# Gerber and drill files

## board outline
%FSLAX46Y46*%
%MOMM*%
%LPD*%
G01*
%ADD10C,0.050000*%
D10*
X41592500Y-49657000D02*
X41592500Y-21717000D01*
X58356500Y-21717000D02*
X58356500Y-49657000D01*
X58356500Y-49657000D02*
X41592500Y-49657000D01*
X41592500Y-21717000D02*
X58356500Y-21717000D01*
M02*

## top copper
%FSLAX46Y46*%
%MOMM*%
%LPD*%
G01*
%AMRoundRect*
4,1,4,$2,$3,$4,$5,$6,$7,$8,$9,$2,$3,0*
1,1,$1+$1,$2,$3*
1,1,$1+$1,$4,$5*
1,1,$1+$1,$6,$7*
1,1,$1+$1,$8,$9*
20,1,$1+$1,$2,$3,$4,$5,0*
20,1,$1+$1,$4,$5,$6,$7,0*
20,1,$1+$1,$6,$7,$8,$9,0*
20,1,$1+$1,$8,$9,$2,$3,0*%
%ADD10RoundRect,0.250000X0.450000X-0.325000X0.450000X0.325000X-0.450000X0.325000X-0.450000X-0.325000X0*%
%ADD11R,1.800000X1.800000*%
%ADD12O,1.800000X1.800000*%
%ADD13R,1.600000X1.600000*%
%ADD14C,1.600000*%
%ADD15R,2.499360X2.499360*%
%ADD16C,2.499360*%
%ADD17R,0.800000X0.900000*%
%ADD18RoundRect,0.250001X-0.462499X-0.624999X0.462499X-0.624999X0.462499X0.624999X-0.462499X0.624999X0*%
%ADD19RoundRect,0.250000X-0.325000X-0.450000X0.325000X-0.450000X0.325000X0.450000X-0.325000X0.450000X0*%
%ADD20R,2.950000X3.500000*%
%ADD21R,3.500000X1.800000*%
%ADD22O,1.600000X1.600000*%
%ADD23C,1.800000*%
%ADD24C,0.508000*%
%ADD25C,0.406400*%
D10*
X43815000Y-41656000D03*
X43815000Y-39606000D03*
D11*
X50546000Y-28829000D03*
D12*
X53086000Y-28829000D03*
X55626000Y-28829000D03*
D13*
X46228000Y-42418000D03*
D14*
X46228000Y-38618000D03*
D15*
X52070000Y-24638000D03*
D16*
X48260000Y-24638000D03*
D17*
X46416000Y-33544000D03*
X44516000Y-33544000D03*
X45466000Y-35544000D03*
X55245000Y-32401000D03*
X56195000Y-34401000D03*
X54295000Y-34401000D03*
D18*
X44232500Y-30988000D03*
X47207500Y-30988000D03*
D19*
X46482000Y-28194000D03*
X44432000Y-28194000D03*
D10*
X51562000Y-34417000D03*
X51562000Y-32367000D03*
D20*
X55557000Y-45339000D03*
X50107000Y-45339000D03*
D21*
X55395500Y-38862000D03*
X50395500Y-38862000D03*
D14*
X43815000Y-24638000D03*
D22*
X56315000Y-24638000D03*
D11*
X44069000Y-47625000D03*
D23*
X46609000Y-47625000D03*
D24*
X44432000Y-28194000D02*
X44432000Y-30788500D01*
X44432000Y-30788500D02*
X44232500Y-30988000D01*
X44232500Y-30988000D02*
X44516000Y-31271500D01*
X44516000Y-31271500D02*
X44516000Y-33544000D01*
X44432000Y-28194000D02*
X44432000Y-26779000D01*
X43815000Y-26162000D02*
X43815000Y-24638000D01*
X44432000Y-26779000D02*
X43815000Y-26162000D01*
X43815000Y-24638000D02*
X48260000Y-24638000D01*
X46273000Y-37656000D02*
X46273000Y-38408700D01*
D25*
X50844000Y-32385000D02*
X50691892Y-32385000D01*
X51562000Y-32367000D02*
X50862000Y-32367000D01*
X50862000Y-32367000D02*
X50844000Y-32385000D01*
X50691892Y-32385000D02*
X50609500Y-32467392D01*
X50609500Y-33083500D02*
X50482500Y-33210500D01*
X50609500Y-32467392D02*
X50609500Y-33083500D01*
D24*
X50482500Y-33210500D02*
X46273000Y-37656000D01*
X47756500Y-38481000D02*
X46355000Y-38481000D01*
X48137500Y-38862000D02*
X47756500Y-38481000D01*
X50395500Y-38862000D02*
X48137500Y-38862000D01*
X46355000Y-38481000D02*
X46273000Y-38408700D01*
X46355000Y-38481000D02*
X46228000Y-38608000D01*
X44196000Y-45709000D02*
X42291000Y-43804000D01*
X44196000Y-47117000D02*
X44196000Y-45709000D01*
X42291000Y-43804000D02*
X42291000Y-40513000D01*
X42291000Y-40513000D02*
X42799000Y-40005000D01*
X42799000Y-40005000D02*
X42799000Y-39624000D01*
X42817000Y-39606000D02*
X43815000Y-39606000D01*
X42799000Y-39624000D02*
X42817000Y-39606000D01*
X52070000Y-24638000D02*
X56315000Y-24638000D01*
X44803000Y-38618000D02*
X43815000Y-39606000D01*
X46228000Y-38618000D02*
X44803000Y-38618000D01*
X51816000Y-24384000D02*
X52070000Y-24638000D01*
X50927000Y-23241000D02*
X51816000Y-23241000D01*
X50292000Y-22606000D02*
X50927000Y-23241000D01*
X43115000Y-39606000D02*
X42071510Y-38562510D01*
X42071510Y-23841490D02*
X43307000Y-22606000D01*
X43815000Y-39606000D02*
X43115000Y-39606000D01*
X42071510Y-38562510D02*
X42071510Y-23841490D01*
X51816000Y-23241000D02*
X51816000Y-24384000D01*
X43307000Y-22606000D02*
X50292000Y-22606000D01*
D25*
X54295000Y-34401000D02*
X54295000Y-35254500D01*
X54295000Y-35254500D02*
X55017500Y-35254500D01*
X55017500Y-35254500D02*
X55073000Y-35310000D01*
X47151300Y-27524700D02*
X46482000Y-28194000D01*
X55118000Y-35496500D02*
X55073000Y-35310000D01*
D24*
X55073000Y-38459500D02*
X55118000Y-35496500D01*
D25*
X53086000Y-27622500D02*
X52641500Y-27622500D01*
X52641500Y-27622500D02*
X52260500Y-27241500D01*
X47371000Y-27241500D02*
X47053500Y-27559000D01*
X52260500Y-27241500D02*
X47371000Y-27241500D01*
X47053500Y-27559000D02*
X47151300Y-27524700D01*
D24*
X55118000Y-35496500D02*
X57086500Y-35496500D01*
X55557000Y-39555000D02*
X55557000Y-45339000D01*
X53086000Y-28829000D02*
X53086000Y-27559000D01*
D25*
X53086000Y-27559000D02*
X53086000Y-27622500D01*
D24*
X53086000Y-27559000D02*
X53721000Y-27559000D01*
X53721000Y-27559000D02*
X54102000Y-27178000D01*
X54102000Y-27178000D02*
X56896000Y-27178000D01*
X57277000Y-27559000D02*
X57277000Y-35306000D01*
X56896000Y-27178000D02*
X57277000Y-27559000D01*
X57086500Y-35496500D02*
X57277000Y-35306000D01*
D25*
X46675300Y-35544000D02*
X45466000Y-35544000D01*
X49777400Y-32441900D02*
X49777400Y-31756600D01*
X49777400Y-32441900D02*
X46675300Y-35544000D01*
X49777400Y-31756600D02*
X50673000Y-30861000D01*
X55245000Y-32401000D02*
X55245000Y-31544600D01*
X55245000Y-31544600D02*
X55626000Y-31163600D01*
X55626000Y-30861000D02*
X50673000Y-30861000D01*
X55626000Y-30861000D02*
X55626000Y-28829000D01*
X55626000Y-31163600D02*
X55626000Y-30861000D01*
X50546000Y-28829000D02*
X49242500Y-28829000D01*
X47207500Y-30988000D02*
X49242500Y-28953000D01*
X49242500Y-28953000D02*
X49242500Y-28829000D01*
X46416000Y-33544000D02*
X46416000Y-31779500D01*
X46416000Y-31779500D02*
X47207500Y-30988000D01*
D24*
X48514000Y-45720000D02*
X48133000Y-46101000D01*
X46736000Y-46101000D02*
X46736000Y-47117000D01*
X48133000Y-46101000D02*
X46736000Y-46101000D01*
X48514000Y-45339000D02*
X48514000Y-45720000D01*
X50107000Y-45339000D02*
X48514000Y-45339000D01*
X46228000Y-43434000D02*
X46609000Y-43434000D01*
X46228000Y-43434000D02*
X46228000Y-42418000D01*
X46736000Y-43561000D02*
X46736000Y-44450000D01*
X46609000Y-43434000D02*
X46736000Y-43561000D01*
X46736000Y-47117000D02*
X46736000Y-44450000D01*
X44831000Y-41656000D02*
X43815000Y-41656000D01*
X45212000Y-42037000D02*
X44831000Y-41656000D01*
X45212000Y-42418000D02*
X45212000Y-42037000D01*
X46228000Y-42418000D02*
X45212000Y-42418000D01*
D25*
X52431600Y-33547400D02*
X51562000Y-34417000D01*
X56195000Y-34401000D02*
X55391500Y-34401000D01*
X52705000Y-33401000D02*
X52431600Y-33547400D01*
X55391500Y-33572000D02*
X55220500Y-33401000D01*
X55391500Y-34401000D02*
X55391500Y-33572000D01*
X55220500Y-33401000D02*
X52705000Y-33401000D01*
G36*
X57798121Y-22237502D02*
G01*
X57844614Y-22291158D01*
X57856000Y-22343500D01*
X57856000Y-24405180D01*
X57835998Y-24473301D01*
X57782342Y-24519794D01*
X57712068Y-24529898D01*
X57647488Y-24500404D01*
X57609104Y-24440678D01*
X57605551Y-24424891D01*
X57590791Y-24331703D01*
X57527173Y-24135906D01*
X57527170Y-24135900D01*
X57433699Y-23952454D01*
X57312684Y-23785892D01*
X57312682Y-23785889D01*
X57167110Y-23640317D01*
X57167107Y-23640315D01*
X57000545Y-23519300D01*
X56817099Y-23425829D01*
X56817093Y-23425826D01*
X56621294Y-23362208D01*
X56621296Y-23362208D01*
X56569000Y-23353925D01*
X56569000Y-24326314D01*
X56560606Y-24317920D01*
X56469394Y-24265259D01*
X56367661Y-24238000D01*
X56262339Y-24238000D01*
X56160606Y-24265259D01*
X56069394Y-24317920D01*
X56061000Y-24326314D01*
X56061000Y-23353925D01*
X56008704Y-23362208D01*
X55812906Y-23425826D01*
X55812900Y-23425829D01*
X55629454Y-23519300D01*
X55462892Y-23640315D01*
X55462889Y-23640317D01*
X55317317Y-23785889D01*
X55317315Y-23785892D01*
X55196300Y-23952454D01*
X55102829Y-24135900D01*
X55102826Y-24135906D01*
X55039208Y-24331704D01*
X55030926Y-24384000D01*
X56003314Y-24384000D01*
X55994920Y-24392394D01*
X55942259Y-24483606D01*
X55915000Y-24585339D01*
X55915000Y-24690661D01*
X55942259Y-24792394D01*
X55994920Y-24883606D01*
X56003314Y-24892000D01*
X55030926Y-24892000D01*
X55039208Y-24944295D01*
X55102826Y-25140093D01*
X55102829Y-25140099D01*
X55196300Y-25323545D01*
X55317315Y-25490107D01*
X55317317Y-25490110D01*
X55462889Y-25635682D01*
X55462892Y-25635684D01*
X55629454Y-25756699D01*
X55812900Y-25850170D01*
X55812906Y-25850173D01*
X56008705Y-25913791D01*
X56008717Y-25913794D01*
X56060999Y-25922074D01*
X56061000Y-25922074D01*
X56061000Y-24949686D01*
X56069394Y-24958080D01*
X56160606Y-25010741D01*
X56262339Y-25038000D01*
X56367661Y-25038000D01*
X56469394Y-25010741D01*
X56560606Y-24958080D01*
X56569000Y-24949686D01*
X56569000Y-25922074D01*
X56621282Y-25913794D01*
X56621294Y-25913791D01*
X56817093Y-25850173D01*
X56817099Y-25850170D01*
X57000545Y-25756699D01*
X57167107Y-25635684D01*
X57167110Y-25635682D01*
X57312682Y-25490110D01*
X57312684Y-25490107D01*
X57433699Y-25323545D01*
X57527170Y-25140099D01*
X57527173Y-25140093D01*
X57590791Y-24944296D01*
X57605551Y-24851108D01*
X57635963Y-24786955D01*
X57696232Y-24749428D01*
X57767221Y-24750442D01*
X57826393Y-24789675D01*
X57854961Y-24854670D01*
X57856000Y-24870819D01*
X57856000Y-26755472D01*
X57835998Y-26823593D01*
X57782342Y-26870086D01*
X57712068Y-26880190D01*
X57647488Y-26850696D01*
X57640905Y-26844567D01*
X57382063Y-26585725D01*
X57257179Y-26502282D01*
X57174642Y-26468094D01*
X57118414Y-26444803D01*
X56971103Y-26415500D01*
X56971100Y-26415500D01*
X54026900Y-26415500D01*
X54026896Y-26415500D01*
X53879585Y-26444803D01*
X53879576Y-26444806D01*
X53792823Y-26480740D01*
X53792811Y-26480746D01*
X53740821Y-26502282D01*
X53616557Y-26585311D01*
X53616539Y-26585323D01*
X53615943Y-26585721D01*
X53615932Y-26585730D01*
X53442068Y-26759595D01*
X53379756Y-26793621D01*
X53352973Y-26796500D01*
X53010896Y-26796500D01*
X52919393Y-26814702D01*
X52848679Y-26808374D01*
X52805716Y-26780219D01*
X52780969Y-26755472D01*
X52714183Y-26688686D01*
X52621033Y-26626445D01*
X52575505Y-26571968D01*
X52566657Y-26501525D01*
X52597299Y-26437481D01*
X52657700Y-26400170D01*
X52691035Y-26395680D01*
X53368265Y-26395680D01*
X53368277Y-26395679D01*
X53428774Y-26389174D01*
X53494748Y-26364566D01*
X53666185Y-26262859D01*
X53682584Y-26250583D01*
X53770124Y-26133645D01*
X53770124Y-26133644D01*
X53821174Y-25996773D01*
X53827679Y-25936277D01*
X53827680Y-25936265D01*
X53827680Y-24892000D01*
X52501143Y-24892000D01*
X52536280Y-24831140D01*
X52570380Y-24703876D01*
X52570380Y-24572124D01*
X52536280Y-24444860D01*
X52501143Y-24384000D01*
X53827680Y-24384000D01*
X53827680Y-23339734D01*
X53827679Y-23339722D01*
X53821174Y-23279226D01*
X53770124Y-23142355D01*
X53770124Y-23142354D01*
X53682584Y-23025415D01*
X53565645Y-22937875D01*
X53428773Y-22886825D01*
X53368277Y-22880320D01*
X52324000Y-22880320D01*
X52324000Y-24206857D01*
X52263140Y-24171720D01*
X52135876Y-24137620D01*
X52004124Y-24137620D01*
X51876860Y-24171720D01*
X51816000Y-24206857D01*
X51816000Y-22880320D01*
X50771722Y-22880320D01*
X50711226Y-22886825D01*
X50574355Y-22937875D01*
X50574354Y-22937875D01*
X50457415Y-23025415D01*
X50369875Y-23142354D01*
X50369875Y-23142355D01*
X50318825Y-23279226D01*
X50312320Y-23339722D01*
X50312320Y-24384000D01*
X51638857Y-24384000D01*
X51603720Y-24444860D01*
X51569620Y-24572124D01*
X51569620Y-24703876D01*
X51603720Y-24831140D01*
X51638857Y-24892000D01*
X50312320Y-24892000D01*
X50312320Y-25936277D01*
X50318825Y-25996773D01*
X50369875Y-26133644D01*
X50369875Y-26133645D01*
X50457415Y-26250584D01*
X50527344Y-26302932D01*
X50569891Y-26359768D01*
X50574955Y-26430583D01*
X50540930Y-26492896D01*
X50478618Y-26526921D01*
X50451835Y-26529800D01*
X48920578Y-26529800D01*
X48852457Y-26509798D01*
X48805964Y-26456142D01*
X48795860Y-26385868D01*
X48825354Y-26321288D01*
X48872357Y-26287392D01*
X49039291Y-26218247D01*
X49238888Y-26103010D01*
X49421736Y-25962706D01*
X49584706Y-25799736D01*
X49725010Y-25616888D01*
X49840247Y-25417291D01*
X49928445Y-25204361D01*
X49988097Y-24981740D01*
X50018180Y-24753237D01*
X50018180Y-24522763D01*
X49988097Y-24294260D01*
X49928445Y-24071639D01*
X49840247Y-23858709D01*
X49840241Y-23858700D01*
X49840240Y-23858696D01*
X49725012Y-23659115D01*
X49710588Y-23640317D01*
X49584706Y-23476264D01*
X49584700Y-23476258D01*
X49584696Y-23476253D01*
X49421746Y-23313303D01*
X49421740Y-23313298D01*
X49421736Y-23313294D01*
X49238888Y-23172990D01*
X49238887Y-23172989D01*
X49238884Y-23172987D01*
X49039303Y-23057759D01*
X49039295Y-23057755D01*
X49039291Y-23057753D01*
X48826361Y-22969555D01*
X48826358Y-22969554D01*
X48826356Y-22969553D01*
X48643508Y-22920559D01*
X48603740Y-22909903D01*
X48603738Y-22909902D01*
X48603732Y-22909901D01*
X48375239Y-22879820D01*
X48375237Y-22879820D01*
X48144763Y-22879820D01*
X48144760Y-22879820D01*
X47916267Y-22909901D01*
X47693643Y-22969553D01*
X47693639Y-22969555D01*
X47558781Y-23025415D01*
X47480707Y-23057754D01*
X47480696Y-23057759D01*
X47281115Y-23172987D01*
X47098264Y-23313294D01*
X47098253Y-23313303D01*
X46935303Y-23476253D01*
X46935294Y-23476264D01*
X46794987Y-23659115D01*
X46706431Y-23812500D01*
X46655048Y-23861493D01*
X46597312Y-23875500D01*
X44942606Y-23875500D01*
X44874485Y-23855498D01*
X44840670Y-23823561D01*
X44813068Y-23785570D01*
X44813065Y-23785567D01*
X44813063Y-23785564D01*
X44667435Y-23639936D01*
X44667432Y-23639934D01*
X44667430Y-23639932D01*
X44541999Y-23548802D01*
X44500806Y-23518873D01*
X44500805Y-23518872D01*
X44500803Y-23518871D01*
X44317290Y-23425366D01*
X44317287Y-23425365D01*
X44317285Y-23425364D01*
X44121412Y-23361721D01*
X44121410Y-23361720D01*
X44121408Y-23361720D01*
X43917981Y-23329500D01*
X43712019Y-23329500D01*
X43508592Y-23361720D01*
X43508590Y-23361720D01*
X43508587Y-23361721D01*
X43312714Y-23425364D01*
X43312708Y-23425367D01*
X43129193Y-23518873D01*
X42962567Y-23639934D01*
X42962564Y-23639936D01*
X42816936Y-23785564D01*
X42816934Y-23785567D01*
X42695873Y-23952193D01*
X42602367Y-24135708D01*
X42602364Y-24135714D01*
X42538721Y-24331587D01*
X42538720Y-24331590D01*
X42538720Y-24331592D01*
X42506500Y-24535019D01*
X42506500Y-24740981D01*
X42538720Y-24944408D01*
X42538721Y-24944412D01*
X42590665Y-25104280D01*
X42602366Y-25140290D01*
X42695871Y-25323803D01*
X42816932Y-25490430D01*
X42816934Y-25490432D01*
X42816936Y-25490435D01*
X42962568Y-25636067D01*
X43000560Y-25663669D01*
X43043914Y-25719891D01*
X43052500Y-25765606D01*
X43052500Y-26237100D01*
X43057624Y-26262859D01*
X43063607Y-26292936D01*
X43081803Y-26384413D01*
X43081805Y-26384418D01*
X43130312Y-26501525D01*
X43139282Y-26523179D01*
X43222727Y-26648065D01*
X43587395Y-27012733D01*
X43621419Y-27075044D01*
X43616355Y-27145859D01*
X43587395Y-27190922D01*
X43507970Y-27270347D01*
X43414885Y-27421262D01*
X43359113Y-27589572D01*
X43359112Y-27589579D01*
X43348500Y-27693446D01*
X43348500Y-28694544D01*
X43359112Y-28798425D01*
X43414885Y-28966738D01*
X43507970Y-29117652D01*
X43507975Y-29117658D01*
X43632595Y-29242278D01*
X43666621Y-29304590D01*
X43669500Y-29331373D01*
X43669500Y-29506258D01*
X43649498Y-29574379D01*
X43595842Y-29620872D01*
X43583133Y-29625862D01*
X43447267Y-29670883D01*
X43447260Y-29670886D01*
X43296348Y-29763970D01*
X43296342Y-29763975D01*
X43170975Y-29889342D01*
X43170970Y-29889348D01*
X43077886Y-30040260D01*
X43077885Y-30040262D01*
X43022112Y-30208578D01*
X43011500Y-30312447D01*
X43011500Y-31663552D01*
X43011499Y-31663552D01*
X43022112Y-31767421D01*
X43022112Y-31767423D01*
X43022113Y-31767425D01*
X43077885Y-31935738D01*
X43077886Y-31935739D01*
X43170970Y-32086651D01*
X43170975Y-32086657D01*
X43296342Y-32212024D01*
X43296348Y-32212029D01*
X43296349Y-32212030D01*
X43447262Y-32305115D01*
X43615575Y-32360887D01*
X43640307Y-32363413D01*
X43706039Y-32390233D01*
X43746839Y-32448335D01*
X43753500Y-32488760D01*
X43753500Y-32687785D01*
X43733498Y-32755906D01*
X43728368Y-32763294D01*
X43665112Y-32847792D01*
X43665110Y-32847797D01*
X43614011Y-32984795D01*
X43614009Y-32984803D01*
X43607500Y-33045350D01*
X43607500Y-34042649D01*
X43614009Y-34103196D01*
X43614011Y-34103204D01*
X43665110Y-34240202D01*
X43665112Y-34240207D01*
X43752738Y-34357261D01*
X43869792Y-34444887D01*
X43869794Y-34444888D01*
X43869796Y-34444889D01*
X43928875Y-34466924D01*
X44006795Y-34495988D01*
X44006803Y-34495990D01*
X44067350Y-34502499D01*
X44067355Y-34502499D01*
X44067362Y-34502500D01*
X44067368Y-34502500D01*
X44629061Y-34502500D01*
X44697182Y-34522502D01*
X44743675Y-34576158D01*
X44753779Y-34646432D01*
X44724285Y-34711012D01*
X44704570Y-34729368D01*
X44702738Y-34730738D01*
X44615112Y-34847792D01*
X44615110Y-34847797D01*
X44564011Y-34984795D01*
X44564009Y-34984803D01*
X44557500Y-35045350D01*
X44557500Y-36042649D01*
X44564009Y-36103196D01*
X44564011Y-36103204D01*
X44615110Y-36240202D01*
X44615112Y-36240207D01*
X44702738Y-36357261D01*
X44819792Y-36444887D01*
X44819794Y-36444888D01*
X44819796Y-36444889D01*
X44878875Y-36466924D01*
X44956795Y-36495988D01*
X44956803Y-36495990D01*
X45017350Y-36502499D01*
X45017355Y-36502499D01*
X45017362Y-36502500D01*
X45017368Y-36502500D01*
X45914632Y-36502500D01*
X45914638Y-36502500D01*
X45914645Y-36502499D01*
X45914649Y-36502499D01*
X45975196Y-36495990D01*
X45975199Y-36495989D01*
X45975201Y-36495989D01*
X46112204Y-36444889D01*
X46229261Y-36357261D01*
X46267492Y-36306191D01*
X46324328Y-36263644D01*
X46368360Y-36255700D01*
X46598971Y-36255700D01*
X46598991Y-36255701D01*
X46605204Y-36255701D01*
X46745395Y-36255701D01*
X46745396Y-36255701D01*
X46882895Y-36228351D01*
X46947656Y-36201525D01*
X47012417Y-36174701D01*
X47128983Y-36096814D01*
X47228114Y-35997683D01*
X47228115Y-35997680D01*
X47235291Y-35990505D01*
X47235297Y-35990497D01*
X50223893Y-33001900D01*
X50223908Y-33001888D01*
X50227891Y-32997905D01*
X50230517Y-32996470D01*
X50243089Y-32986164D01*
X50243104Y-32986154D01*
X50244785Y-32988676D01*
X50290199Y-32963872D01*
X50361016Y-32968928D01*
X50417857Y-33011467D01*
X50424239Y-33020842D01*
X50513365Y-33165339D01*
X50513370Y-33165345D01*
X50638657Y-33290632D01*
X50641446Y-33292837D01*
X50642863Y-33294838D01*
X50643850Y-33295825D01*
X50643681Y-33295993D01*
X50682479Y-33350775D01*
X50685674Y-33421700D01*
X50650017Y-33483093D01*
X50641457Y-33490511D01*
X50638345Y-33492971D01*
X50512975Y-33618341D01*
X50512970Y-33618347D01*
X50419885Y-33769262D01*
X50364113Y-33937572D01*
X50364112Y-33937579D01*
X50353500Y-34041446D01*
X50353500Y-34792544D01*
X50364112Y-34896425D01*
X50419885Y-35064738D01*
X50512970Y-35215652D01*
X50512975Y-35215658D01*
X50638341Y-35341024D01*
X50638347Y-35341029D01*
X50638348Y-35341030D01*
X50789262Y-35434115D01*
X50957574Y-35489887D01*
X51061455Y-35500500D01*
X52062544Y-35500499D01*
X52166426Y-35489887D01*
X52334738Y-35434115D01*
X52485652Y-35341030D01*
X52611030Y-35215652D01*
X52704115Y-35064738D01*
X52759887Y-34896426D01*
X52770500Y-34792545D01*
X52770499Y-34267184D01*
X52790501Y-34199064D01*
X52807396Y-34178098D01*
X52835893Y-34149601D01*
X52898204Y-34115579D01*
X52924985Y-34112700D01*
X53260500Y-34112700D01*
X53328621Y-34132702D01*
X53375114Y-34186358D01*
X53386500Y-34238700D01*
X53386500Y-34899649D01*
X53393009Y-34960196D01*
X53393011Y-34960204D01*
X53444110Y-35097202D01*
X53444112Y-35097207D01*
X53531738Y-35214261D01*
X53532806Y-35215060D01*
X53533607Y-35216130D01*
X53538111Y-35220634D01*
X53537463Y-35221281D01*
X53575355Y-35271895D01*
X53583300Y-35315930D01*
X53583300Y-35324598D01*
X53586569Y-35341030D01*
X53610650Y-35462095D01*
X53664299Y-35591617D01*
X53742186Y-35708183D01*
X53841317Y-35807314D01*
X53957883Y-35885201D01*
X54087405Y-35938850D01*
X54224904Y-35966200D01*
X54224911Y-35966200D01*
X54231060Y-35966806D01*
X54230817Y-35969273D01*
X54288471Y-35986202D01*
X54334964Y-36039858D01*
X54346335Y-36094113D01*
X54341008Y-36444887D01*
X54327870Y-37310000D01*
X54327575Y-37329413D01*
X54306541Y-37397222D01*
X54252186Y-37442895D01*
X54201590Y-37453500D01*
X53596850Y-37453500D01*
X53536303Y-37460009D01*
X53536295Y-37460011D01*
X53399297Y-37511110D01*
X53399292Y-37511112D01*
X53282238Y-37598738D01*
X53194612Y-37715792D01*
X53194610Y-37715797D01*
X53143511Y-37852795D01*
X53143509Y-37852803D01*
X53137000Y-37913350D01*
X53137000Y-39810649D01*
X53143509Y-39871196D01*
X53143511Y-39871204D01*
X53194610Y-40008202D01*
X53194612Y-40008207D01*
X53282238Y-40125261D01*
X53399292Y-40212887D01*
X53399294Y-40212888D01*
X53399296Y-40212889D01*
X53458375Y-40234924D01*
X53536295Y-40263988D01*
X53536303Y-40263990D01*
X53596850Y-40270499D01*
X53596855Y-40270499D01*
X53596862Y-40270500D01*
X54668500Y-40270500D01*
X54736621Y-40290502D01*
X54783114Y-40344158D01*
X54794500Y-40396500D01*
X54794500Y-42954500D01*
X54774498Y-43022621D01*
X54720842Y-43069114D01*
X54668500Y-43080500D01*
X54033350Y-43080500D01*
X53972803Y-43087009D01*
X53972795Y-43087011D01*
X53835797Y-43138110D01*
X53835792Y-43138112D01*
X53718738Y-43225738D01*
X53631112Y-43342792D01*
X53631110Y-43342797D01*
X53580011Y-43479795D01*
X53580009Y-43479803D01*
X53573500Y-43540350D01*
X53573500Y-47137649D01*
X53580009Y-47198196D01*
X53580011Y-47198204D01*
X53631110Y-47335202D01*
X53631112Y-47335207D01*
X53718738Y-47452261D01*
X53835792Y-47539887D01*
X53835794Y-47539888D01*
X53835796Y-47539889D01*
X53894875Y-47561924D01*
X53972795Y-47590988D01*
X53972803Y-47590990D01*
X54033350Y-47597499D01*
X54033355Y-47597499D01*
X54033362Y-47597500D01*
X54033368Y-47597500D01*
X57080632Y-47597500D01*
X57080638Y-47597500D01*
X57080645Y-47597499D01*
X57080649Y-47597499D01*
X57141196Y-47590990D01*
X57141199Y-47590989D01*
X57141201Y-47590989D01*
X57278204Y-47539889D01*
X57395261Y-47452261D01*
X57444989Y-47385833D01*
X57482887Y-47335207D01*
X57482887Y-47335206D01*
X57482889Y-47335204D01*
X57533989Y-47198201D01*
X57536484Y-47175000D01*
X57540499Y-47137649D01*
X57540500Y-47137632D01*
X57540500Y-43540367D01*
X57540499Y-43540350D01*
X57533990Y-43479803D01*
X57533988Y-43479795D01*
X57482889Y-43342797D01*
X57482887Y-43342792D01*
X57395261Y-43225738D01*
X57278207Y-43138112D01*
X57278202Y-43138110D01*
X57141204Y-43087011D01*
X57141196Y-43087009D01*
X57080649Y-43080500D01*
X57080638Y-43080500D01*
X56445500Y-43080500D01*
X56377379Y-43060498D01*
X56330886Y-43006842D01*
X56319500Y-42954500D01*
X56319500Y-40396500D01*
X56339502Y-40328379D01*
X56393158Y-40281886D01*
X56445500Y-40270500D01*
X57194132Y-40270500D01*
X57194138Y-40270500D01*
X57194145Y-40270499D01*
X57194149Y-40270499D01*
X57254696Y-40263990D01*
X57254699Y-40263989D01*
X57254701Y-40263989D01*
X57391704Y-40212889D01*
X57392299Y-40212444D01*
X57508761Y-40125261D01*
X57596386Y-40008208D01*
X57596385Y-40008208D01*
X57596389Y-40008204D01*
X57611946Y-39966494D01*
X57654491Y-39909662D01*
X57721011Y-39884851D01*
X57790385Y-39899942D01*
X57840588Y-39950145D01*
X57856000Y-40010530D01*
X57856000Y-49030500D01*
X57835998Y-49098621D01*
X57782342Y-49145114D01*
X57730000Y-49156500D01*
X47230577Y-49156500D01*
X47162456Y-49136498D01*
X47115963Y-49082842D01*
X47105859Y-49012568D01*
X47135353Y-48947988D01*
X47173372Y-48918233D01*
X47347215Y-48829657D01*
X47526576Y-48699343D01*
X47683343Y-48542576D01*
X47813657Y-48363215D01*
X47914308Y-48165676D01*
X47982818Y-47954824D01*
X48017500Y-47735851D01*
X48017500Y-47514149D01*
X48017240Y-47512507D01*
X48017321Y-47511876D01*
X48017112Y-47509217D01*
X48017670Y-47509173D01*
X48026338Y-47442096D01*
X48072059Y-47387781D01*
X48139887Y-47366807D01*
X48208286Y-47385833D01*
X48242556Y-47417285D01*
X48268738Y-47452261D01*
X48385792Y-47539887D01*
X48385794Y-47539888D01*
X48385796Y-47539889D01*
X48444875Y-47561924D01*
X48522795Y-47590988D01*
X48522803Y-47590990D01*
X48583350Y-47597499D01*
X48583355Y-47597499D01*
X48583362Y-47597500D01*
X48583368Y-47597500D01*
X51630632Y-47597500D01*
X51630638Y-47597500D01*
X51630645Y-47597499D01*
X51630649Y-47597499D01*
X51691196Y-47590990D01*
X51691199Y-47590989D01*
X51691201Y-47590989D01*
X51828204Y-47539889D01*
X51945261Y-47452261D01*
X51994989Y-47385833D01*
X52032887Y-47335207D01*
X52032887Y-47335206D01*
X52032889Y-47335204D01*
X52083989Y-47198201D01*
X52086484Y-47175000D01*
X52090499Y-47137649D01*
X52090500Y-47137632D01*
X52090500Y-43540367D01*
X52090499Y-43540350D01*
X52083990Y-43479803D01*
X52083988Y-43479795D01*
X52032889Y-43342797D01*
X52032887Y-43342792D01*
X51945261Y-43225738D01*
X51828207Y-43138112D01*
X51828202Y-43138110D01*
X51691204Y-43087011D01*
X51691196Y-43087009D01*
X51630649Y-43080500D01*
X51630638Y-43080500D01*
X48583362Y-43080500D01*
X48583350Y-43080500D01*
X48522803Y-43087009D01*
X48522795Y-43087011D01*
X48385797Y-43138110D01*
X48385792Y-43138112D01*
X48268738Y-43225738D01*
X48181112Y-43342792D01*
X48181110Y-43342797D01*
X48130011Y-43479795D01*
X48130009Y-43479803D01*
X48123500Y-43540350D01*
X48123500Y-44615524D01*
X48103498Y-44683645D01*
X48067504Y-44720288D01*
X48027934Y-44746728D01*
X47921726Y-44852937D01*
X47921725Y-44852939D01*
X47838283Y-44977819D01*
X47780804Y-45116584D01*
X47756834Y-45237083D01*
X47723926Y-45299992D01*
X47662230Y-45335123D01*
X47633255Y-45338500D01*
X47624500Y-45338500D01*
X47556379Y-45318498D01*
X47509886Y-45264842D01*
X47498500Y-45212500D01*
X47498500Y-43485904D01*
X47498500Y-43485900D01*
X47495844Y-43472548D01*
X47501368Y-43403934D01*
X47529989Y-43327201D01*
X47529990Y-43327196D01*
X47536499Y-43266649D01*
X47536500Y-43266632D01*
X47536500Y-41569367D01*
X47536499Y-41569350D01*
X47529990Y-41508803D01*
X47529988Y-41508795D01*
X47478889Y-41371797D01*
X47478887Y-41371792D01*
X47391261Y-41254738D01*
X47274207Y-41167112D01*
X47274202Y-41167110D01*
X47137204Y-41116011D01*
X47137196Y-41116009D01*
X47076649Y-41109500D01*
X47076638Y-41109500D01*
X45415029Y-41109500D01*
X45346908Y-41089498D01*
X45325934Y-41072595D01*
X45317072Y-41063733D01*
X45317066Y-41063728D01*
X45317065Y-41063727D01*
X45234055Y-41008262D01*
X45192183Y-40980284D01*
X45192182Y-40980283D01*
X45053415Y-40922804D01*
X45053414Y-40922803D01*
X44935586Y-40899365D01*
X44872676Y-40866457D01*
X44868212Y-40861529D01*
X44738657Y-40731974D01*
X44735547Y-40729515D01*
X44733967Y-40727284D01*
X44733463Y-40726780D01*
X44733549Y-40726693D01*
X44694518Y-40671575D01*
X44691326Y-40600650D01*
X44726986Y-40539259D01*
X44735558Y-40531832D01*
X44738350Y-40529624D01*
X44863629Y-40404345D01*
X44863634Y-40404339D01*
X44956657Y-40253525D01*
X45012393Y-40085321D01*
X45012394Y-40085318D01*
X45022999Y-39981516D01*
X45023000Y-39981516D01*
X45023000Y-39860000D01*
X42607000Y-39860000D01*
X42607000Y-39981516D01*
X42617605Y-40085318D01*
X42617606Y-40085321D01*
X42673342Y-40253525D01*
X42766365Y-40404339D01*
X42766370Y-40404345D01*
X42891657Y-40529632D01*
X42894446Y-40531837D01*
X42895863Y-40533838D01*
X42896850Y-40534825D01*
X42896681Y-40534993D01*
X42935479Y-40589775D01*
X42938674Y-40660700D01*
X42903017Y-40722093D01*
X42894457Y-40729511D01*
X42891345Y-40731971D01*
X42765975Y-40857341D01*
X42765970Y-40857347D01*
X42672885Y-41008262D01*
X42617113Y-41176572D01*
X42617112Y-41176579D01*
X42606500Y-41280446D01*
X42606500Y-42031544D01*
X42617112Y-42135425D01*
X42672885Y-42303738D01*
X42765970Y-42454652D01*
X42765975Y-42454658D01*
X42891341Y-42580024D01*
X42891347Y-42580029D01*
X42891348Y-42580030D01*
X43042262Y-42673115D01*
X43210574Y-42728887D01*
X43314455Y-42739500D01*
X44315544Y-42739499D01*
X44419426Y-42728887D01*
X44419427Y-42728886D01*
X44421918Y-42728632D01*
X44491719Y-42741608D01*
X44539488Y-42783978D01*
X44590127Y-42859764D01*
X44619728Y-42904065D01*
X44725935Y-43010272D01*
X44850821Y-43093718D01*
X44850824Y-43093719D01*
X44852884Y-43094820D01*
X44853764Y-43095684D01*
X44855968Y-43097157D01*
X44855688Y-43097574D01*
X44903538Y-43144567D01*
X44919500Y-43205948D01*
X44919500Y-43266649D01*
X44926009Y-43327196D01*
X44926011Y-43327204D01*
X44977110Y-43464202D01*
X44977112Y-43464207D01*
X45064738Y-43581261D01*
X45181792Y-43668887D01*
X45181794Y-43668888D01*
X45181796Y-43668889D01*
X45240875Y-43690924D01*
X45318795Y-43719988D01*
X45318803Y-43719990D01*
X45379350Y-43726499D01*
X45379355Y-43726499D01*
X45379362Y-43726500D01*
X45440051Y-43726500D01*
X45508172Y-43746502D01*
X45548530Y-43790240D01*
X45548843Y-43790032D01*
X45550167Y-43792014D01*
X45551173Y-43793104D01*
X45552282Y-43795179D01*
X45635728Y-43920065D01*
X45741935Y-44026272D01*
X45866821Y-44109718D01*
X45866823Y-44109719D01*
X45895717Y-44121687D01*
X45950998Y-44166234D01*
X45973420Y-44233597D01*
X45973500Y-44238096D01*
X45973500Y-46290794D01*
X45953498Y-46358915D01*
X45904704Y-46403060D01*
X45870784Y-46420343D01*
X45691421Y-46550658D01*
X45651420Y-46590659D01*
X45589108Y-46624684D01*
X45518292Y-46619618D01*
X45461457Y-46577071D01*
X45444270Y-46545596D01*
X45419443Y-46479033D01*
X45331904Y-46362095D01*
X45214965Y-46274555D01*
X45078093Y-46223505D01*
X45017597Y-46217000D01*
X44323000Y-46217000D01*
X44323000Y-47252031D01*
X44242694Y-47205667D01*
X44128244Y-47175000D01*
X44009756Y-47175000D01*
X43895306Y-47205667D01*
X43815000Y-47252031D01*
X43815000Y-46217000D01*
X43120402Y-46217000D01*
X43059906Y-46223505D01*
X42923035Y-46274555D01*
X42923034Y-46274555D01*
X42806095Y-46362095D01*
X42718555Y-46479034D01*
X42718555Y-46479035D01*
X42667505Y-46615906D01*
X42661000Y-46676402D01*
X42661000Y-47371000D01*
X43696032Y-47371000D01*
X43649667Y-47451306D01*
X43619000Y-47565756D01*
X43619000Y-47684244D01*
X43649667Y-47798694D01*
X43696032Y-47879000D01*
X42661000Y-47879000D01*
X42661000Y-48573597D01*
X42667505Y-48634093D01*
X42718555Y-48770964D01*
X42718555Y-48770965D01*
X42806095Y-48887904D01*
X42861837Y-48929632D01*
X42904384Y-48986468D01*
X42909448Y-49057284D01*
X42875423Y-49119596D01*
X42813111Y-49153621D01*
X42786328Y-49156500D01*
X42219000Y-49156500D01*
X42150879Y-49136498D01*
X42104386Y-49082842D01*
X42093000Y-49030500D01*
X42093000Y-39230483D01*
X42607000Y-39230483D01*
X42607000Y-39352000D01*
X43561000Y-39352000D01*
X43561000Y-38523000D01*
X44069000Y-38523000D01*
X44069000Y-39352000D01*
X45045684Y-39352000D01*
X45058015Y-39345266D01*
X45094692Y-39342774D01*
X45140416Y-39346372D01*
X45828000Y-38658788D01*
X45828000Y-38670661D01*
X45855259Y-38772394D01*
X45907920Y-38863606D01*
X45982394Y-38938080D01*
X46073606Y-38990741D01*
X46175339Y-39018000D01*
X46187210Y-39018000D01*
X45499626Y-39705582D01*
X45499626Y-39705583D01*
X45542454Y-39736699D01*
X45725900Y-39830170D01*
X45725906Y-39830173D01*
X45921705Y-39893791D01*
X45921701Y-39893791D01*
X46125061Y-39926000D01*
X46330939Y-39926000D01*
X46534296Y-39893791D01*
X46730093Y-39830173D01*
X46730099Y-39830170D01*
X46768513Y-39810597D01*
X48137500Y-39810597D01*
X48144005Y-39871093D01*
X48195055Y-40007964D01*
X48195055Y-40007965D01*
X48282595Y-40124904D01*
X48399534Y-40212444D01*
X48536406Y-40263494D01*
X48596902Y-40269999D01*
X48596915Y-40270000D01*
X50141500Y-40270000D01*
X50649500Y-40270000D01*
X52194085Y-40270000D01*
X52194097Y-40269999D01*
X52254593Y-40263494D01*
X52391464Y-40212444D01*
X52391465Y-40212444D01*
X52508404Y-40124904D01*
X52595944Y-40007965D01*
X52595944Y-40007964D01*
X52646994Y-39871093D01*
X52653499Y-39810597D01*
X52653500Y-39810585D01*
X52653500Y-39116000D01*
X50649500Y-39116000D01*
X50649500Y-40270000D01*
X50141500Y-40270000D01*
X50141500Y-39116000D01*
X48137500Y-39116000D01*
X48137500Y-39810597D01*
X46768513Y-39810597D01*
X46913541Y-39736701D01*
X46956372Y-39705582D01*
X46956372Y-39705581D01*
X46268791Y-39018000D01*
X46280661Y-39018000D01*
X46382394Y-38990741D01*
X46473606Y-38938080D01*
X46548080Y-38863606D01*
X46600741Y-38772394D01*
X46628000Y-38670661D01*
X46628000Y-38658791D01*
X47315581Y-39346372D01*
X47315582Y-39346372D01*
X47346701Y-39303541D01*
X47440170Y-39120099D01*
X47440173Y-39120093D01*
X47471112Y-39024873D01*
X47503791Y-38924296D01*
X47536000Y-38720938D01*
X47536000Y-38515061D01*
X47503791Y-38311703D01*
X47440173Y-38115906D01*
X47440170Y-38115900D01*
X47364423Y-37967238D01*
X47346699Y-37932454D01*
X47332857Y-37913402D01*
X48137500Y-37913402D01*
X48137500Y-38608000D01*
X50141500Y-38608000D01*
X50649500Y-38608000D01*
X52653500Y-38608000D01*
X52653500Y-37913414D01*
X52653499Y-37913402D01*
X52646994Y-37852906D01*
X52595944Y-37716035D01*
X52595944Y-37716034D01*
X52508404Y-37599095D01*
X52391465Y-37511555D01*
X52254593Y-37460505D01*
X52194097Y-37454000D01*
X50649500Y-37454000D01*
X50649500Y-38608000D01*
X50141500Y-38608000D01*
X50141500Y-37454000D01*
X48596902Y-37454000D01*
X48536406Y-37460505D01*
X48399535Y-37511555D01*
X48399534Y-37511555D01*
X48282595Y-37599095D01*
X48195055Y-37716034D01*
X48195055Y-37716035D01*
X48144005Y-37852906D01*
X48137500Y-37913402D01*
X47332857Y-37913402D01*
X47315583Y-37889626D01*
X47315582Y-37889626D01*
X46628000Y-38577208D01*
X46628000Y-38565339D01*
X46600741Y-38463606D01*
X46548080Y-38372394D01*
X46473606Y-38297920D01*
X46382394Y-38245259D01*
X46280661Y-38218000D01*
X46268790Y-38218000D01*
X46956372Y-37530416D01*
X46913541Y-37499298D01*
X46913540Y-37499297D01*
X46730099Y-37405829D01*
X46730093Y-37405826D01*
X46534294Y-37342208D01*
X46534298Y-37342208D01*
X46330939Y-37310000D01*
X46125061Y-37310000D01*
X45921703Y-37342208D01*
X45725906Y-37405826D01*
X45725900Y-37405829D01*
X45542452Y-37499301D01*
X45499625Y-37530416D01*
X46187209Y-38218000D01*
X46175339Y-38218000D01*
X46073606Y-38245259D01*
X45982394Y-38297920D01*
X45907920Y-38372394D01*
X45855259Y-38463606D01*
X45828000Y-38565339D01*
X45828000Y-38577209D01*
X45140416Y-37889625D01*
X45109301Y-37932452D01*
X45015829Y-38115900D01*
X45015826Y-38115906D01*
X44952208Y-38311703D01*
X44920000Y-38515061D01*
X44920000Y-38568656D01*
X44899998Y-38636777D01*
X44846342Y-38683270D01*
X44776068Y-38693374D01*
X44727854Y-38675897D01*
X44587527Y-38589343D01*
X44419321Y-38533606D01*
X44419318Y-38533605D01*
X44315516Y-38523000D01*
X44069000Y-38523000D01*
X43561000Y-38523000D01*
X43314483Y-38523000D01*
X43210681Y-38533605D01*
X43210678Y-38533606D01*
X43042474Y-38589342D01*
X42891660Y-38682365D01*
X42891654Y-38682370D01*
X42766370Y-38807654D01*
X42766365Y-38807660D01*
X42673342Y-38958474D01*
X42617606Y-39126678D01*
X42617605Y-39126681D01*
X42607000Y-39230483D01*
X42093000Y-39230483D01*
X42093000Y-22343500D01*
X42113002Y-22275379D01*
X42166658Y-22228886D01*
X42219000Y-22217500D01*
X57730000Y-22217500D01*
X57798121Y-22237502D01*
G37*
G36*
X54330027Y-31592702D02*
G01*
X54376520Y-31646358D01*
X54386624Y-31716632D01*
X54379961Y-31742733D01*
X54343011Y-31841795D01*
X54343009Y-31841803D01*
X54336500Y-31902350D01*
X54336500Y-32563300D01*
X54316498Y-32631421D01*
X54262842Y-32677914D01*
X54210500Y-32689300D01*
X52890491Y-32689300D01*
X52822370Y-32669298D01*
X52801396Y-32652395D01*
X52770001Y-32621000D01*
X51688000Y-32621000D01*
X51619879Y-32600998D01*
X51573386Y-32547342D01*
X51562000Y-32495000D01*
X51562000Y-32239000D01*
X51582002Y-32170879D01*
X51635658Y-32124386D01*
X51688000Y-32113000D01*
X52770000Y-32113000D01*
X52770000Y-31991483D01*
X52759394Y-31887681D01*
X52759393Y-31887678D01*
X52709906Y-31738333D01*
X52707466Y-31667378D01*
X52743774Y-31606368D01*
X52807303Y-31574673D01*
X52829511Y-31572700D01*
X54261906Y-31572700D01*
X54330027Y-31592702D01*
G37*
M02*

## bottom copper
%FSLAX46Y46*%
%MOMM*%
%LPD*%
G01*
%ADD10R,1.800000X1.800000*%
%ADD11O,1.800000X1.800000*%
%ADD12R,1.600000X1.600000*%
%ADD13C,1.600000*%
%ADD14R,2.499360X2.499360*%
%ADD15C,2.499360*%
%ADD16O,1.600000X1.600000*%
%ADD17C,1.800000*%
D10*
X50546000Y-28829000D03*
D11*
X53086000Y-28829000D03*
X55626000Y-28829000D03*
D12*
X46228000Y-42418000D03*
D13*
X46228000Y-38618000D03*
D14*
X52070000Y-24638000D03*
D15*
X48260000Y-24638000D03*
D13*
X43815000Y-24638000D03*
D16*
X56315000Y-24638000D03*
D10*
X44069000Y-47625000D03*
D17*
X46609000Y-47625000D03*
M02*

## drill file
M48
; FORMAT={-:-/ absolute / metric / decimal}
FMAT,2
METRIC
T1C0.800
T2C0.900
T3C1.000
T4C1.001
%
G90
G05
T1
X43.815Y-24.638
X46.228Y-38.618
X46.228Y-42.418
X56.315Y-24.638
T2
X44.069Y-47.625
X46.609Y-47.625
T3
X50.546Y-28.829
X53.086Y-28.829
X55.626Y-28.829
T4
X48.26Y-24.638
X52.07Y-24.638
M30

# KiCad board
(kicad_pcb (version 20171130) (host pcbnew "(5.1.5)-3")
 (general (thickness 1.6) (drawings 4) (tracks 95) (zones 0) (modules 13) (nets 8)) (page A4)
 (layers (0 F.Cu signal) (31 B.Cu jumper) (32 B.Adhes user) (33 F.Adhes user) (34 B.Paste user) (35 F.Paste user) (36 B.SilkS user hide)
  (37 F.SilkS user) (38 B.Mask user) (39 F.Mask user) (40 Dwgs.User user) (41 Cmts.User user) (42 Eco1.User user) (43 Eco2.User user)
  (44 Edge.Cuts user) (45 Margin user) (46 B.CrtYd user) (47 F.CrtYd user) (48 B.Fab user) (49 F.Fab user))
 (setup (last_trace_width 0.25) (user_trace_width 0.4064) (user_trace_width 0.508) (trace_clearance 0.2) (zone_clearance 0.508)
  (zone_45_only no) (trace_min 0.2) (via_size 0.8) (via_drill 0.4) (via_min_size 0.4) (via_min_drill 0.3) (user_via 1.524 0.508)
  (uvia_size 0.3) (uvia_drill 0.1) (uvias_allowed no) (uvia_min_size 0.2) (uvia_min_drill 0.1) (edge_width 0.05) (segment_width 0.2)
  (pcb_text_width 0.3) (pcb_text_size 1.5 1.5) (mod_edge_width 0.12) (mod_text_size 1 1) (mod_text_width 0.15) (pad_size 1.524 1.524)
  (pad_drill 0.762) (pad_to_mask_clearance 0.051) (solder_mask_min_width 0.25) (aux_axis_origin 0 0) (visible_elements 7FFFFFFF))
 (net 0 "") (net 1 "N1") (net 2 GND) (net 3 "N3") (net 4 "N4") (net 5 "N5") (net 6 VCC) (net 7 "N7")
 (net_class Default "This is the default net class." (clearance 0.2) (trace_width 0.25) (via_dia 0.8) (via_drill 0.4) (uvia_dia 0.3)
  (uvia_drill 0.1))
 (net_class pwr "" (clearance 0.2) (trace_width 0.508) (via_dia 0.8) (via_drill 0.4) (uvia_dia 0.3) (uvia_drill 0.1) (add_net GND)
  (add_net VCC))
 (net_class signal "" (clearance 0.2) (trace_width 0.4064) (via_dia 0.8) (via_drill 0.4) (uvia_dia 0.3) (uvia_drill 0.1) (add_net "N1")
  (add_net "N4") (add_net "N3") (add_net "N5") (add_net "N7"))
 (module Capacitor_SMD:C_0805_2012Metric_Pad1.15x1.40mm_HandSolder (layer F.Cu) (at 43.815 40.631 90)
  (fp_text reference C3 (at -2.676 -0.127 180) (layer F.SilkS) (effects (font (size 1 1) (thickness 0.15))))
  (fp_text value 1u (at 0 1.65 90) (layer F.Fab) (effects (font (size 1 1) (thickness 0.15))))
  (pad 1 smd roundrect (at -1.025 0 90) (size 1.15 1.4) (layers F.Cu F.Paste F.Mask) (roundrect_rratio 0.217391) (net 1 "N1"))
  (pad 2 smd roundrect (at 1.025 0 90) (size 1.15 1.4) (layers F.Cu F.Paste F.Mask) (roundrect_rratio 0.217391) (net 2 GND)))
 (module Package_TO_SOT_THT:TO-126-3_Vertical (layer B.Cu) (at 50.546 28.829)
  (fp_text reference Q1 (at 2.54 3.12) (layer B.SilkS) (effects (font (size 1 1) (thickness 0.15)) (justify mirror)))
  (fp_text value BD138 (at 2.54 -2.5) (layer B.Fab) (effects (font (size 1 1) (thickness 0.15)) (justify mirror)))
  (pad 1 thru_hole rect (at 0 0) (size 1.8 1.8) (drill 1) (layers *.Cu *.Mask) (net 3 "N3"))
  (pad 2 thru_hole oval (at 2.54 0) (size 1.8 1.8) (drill 1) (layers *.Cu *.Mask) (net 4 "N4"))
  (pad 3 thru_hole oval (at 5.08 0) (size 1.8 1.8) (drill 1) (layers *.Cu *.Mask) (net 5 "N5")))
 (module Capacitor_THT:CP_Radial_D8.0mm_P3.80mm (layer B.Cu) (at 46.228 42.418 90)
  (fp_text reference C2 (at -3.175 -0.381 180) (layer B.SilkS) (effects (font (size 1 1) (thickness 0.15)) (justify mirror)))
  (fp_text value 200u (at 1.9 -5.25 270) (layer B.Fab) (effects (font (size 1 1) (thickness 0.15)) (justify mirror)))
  (pad 1 thru_hole rect (at 0 0 90) (size 1.6 1.6) (drill 0.8) (layers *.Cu *.Mask) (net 1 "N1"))
  (pad 2 thru_hole circle (at 3.8 0 90) (size 1.6 1.6) (drill 0.8) (layers *.Cu *.Mask) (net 2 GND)))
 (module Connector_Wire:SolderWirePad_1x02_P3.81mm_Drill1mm (layer F.Cu) (at 52.07 24.638 180)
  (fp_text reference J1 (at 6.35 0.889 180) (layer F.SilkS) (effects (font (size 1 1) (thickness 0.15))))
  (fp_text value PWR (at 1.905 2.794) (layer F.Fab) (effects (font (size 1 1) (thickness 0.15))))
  (pad 1 thru_hole rect (at 0 0 180) (size 2.49936 2.49936) (drill 1.00076) (layers *.Cu *.Mask) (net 2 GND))
  (pad 2 thru_hole circle (at 3.81 0 180) (size 2.49936 2.49936) (drill 1.00076) (layers *.Cu *.Mask) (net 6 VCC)))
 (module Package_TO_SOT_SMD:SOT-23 (layer F.Cu) (at 45.466 34.544 270)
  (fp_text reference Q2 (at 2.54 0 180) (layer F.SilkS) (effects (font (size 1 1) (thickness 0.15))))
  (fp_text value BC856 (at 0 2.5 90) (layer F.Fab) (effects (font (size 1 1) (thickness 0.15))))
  (pad 1 smd rect (at -1 -0.95 270) (size 0.9 0.8) (layers F.Cu F.Paste F.Mask) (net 3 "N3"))
  (pad 2 smd rect (at -1 0.95 270) (size 0.9 0.8) (layers F.Cu F.Paste F.Mask) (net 6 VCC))
  (pad 3 smd rect (at 1 0 270) (size 0.9 0.8) (layers F.Cu F.Paste F.Mask) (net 5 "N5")))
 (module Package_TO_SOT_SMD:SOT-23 (layer F.Cu) (at 55.245 33.401 90)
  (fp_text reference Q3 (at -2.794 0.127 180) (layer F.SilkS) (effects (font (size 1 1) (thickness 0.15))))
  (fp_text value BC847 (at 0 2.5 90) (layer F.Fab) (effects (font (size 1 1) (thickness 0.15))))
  (pad 3 smd rect (at 1 0 90) (size 0.9 0.8) (layers F.Cu F.Paste F.Mask) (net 5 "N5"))
  (pad 2 smd rect (at -1 0.95 90) (size 0.9 0.8) (layers F.Cu F.Paste F.Mask) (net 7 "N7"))
  (pad 1 smd rect (at -1 -0.95 90) (size 0.9 0.8) (layers F.Cu F.Paste F.Mask) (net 4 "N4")))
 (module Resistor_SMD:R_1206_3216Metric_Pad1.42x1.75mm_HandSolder (layer F.Cu) (at 45.72 30.988)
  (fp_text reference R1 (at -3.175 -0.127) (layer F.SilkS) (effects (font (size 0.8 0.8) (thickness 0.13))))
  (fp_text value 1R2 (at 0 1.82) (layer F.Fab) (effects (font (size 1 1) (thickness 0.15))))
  (pad 1 smd roundrect (at -1.4875 0) (size 1.425 1.75) (layers F.Cu F.Paste F.Mask) (roundrect_rratio 0.175439) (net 6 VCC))
  (pad 2 smd roundrect (at 1.4875 0) (size 1.425 1.75) (layers F.Cu F.Paste F.Mask) (roundrect_rratio 0.175439) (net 3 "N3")))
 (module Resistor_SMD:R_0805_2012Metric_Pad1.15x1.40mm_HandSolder (layer F.Cu) (at 45.457 28.194)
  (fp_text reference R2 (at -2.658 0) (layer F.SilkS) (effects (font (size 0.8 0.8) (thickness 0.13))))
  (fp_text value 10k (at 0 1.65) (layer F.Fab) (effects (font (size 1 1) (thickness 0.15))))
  (pad 2 smd roundrect (at 1.025 0) (size 1.15 1.4) (layers F.Cu F.Paste F.Mask) (roundrect_rratio 0.217391) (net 4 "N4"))
  (pad 1 smd roundrect (at -1.025 0) (size 1.15 1.4) (layers F.Cu F.Paste F.Mask) (roundrect_rratio 0.217391) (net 6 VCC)))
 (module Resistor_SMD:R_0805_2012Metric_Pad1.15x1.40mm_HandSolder (layer F.Cu) (at 51.562 33.392 90)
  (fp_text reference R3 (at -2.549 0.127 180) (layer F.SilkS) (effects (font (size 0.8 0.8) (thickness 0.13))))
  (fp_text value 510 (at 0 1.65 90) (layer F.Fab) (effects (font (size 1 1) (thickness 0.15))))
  (pad 1 smd roundrect (at -1.025 0 90) (size 1.15 1.4) (layers F.Cu F.Paste F.Mask) (roundrect_rratio 0.217391) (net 7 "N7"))
  (pad 2 smd roundrect (at 1.025 0 90) (size 1.15 1.4) (layers F.Cu F.Paste F.Mask) (roundrect_rratio 0.217391) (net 2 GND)))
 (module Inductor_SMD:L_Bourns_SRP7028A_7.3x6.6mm (layer F.Cu) (at 52.832 45.339 180)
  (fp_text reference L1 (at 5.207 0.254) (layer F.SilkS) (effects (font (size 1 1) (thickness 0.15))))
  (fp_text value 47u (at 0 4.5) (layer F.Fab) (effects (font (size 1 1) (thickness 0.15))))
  (pad 1 smd rect (at -2.725 0 180) (size 2.95 3.5) (layers F.Cu F.Paste F.Mask) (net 4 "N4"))
  (pad 2 smd rect (at 2.725 0 180) (size 2.95 3.5) (layers F.Cu F.Paste F.Mask) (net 1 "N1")))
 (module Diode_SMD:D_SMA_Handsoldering (layer F.Cu) (at 52.8955 38.862 180)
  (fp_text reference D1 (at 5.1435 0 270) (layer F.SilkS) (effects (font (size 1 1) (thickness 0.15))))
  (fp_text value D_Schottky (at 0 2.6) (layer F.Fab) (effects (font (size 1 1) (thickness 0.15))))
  (pad 1 smd rect (at -2.5 0 180) (size 3.5 1.8) (layers F.Cu F.Paste F.Mask) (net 4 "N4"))
  (pad 2 smd rect (at 2.5 0 180) (size 3.5 1.8) (layers F.Cu F.Paste F.Mask) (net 2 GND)))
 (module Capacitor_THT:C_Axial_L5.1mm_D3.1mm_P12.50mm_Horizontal (layer B.Cu) (at 43.815 24.638)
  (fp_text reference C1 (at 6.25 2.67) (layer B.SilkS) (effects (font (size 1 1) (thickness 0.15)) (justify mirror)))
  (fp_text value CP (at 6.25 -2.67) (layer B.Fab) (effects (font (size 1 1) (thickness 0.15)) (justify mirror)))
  (pad 1 thru_hole circle (at 0 0) (size 1.6 1.6) (drill 0.8) (layers *.Cu *.Mask) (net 6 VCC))
  (pad 2 thru_hole oval (at 12.5 0) (size 1.6 1.6) (drill 0.8) (layers *.Cu *.Mask) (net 2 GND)))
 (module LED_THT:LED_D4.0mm (layer B.Cu) (at 44.069 47.625)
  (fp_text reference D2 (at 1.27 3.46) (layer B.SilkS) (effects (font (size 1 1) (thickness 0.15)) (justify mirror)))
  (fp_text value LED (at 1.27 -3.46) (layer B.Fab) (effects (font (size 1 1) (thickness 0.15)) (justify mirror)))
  (pad 1 thru_hole rect (at 0 0) (size 1.8 1.8) (drill 0.9) (layers *.Cu *.Mask) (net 2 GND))
  (pad 2 thru_hole circle (at 2.54 0) (size 1.8 1.8) (drill 0.9) (layers *.Cu *.Mask) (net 1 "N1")))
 (gr_line (start 41.5925 49.657) (end 41.5925 21.717) (layer Edge.Cuts) (width 0.05))
 (gr_line (start 58.3565 21.717) (end 58.3565 49.657) (layer Edge.Cuts) (width 0.05))
 (gr_line (start 58.3565 49.657) (end 41.5925 49.657) (layer Edge.Cuts) (width 0.05))
 (gr_line (start 41.5925 21.717) (end 58.3565 21.717) (layer Edge.Cuts) (width 0.05))
 (segment (start 44.432 28.194) (end 44.432 30.7885) (width 0.508) (layer F.Cu) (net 6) (status 30))
 (segment (start 44.432 30.7885) (end 44.2325 30.988) (width 0.508) (layer F.Cu) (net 6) (status 30))
 (segment (start 44.2325 30.988) (end 44.516 31.2715) (width 0.508) (layer F.Cu) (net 6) (status 30))
 (segment (start 44.516 31.2715) (end 44.516 33.544) (width 0.508) (layer F.Cu) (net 6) (status 30))
 (segment (start 44.432 28.194) (end 44.432 26.779) (width 0.508) (layer F.Cu) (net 6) (status 10))
 (segment (start 43.815 26.162) (end 43.815 24.638) (width 0.508) (layer F.Cu) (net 6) (status 20))
 (segment (start 44.432 26.779) (end 43.815 26.162) (width 0.508) (layer F.Cu) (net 6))
 (segment (start 43.815 24.638) (end 48.26 24.638) (width 0.508) (layer F.Cu) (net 6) (status 30))
 (segment (start 46.273 37.656) (end 46.273 38.4087) (width 0.508) (layer F.Cu) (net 2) (status 20))
 (segment (start 50.844 32.385) (end 50.691892 32.385) (width 0.4064) (layer F.Cu) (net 2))
 (segment (start 51.562 32.367) (end 50.862 32.367) (width 0.4064) (layer F.Cu) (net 2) (status 30))
 (segment (start 50.862 32.367) (end 50.844 32.385) (width 0.4064) (layer F.Cu) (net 2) (status 10))
 (segment (start 50.691892 32.385) (end 50.6095 32.467392) (width 0.4064) (layer F.Cu) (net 2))
 (segment (start 50.6095 33.0835) (end 50.4825 33.2105) (width 0.4064) (layer F.Cu) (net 2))
 (segment (start 50.6095 32.467392) (end 50.6095 33.0835) (width 0.4064) (layer F.Cu) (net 2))
 (segment (start 50.4825 33.2105) (end 46.273 37.656) (width 0.508) (layer F.Cu) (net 2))
 (segment (start 47.7565 38.481) (end 46.355 38.481) (width 0.508) (layer F.Cu) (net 2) (status 20))
 (segment (start 48.1375 38.862) (end 47.7565 38.481) (width 0.508) (layer F.Cu) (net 2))
 (segment (start 50.3955 38.862) (end 48.1375 38.862) (width 0.508) (layer F.Cu) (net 2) (status 10))
 (segment (start 46.355 38.481) (end 46.273 38.4087) (width 0.508) (layer F.Cu) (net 2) (status 30))
 (segment (start 46.355 38.481) (end 46.228 38.608) (width 0.508) (layer F.Cu) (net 2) (status 30))
 (segment (start 44.196 45.709) (end 42.291 43.804) (width 0.508) (layer F.Cu) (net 2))
 (segment (start 44.196 47.117) (end 44.196 45.709) (width 0.508) (layer F.Cu) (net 2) (status 10))
 (segment (start 42.291 43.804) (end 42.291 40.513) (width 0.508) (layer F.Cu) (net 2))
 (segment (start 42.291 40.513) (end 42.799 40.005) (width 0.508) (layer F.Cu) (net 2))
 (segment (start 42.799 40.005) (end 42.799 39.624) (width 0.508) (layer F.Cu) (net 2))
 (segment (start 42.817 39.606) (end 43.815 39.606) (width 0.508) (layer F.Cu) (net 2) (status 20))
 (segment (start 42.799 39.624) (end 42.817 39.606) (width 0.508) (layer F.Cu) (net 2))
 (segment (start 52.07 24.638) (end 56.315 24.638) (width 0.508) (layer F.Cu) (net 2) (status 30))
 (segment (start 44.803 38.618) (end 43.815 39.606) (width 0.508) (layer F.Cu) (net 2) (status 20))
 (segment (start 46.228 38.618) (end 44.803 38.618) (width 0.508) (layer F.Cu) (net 2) (status 10))
 (segment (start 51.816 24.384) (end 52.07 24.638) (width 0.508) (layer F.Cu) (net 2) (status 30))
 (segment (start 50.927 23.241) (end 51.816 23.241) (width 0.508) (layer F.Cu) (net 2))
 (segment (start 50.292 22.606) (end 50.927 23.241) (width 0.508) (layer F.Cu) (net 2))
 (segment (start 43.115 39.606) (end 42.07151 38.56251) (width 0.508) (layer F.Cu) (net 2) (status 10))
 (segment (start 42.07151 23.84149) (end 43.307 22.606) (width 0.508) (layer F.Cu) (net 2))
 (segment (start 43.815 39.606) (end 43.115 39.606) (width 0.508) (layer F.Cu) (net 2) (status 30))
 (segment (start 42.07151 38.56251) (end 42.07151 23.84149) (width 0.508) (layer F.Cu) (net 2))
 (segment (start 51.816 23.241) (end 51.816 24.384) (width 0.508) (layer F.Cu) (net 2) (status 20))
 (segment (start 43.307 22.606) (end 50.292 22.606) (width 0.508) (layer F.Cu) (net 2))
 (segment (start 54.295 34.401) (end 54.295 35.2545) (width 0.4064) (layer F.Cu) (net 4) (status 10))
 (segment (start 54.295 35.2545) (end 55.0175 35.2545) (width 0.4064) (layer F.Cu) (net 4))
 (segment (start 55.0175 35.2545) (end 55.073 35.31) (width 0.4064) (layer F.Cu) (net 4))
 (segment (start 47.1513 27.5247) (end 46.482 28.194) (width 0.4064) (layer F.Cu) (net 4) (status 20))
 (segment (start 55.118 35.4965) (end 55.073 35.31) (width 0.4064) (layer F.Cu) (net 4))
 (segment (start 55.073 38.4595) (end 55.118 35.4965) (width 0.508) (layer F.Cu) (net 4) (status 10))
 (segment (start 53.086 27.6225) (end 52.6415 27.6225) (width 0.4064) (layer F.Cu) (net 4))
 (segment (start 52.6415 27.6225) (end 52.2605 27.2415) (width 0.4064) (layer F.Cu) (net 4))
 (segment (start 47.371 27.2415) (end 47.0535 27.559) (width 0.4064) (layer F.Cu) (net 4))
 (segment (start 52.2605 27.2415) (end 47.371 27.2415) (width 0.4064) (layer F.Cu) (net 4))
 (segment (start 47.0535 27.559) (end 47.1513 27.5247) (width 0.4064) (layer F.Cu) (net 4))
 (segment (start 55.118 35.4965) (end 57.0865 35.4965) (width 0.508) (layer F.Cu) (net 4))
 (segment (start 55.557 39.555) (end 55.557 45.339) (width 0.508) (layer F.Cu) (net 4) (status 30))
 (segment (start 53.086 28.829) (end 53.086 27.559) (width 0.508) (layer F.Cu) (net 4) (status 10))
 (segment (start 53.086 27.559) (end 53.086 27.6225) (width 0.4064) (layer F.Cu) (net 4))
 (segment (start 53.086 27.559) (end 53.721 27.559) (width 0.508) (layer F.Cu) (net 4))
 (segment (start 53.721 27.559) (end 54.102 27.178) (width 0.508) (layer F.Cu) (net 4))
 (segment (start 54.102 27.178) (end 56.896 27.178) (width 0.508) (layer F.Cu) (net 4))
 (segment (start 57.277 27.559) (end 57.277 35.306) (width 0.508) (layer F.Cu) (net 4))
 (segment (start 56.896 27.178) (end 57.277 27.559) (width 0.508) (layer F.Cu) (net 4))
 (segment (start 57.0865 35.4965) (end 57.277 35.306) (width 0.508) (layer F.Cu) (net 4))
 (segment (start 46.6753 35.544) (end 45.466 35.544) (width 0.4064) (layer F.Cu) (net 5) (status 20))
 (segment (start 49.7774 32.4419) (end 49.7774 31.7566) (width 0.4064) (layer F.Cu) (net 5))
 (segment (start 49.7774 32.4419) (end 46.6753 35.544) (width 0.4064) (layer F.Cu) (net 5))
 (segment (start 49.7774 31.7566) (end 50.673 30.861) (width 0.4064) (layer F.Cu) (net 5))
 (segment (start 55.245 32.401) (end 55.245 31.5446) (width 0.4064) (layer F.Cu) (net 5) (status 10))
 (segment (start 55.245 31.5446) (end 55.626 31.1636) (width 0.4064) (layer F.Cu) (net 5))
 (segment (start 55.626 30.861) (end 50.673 30.861) (width 0.4064) (layer F.Cu) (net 5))
 (segment (start 55.626 30.861) (end 55.626 28.829) (width 0.4064) (layer F.Cu) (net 5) (status 20))
 (segment (start 55.626 31.1636) (end 55.626 30.861) (width 0.4064) (layer F.Cu) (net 5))
 (segment (start 50.546 28.829) (end 49.2425 28.829) (width 0.4064) (layer F.Cu) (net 3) (status 10))
 (segment (start 47.2075 30.988) (end 49.2425 28.953) (width 0.4064) (layer F.Cu) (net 3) (status 10))
 (segment (start 49.2425 28.953) (end 49.2425 28.829) (width 0.4064) (layer F.Cu) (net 3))
 (segment (start 46.416 33.544) (end 46.416 31.7795) (width 0.4064) (layer F.Cu) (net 3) (status 10))
 (segment (start 46.416 31.7795) (end 47.2075 30.988) (width 0.4064) (layer F.Cu) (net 3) (status 20))
 (segment (start 48.514 45.72) (end 48.133 46.101) (width 0.508) (layer F.Cu) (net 1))
 (segment (start 46.736 46.101) (end 46.736 47.117) (width 0.508) (layer F.Cu) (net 1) (status 20))
 (segment (start 48.133 46.101) (end 46.736 46.101) (width 0.508) (layer F.Cu) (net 1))
 (segment (start 48.514 45.339) (end 48.514 45.72) (width 0.508) (layer F.Cu) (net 1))
 (segment (start 50.107 45.339) (end 48.514 45.339) (width 0.508) (layer F.Cu) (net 1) (status 10))
 (segment (start 46.228 43.434) (end 46.609 43.434) (width 0.508) (layer F.Cu) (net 1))
 (segment (start 46.228 43.434) (end 46.228 42.418) (width 0.508) (layer F.Cu) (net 1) (status 20))
 (segment (start 46.736 43.561) (end 46.736 44.45) (width 0.508) (layer F.Cu) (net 1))
 (segment (start 46.609 43.434) (end 46.736 43.561) (width 0.508) (layer F.Cu) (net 1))
 (segment (start 46.736 47.117) (end 46.736 44.45) (width 0.508) (layer F.Cu) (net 1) (status 10))
 (segment (start 44.831 41.656) (end 43.815 41.656) (width 0.508) (layer F.Cu) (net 1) (status 20))
 (segment (start 45.212 42.037) (end 44.831 41.656) (width 0.508) (layer F.Cu) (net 1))
 (segment (start 45.212 42.418) (end 45.212 42.037) (width 0.508) (layer F.Cu) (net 1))
 (segment (start 46.228 42.418) (end 45.212 42.418) (width 0.508) (layer F.Cu) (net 1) (status 10))
 (segment (start 52.4316 33.5474) (end 51.562 34.417) (width 0.4064) (layer F.Cu) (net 7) (status 20))
 (segment (start 56.195 34.401) (end 55.3915 34.401) (width 0.4064) (layer F.Cu) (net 7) (status 10))
 (segment (start 52.705 33.401) (end 52.4316 33.5474) (width 0.4064) (layer F.Cu) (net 7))
 (segment (start 55.3915 33.572) (end 55.2205 33.401) (width 0.4064) (layer F.Cu) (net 7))
 (segment (start 55.3915 34.401) (end 55.3915 33.572) (width 0.4064) (layer F.Cu) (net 7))
 (segment (start 55.2205 33.401) (end 52.705 33.401) (width 0.4064) (layer F.Cu) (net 7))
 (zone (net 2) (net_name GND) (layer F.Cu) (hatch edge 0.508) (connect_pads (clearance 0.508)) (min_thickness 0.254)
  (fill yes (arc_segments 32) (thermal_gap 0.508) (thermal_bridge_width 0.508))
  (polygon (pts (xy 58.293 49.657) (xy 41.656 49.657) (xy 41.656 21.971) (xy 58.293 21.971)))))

